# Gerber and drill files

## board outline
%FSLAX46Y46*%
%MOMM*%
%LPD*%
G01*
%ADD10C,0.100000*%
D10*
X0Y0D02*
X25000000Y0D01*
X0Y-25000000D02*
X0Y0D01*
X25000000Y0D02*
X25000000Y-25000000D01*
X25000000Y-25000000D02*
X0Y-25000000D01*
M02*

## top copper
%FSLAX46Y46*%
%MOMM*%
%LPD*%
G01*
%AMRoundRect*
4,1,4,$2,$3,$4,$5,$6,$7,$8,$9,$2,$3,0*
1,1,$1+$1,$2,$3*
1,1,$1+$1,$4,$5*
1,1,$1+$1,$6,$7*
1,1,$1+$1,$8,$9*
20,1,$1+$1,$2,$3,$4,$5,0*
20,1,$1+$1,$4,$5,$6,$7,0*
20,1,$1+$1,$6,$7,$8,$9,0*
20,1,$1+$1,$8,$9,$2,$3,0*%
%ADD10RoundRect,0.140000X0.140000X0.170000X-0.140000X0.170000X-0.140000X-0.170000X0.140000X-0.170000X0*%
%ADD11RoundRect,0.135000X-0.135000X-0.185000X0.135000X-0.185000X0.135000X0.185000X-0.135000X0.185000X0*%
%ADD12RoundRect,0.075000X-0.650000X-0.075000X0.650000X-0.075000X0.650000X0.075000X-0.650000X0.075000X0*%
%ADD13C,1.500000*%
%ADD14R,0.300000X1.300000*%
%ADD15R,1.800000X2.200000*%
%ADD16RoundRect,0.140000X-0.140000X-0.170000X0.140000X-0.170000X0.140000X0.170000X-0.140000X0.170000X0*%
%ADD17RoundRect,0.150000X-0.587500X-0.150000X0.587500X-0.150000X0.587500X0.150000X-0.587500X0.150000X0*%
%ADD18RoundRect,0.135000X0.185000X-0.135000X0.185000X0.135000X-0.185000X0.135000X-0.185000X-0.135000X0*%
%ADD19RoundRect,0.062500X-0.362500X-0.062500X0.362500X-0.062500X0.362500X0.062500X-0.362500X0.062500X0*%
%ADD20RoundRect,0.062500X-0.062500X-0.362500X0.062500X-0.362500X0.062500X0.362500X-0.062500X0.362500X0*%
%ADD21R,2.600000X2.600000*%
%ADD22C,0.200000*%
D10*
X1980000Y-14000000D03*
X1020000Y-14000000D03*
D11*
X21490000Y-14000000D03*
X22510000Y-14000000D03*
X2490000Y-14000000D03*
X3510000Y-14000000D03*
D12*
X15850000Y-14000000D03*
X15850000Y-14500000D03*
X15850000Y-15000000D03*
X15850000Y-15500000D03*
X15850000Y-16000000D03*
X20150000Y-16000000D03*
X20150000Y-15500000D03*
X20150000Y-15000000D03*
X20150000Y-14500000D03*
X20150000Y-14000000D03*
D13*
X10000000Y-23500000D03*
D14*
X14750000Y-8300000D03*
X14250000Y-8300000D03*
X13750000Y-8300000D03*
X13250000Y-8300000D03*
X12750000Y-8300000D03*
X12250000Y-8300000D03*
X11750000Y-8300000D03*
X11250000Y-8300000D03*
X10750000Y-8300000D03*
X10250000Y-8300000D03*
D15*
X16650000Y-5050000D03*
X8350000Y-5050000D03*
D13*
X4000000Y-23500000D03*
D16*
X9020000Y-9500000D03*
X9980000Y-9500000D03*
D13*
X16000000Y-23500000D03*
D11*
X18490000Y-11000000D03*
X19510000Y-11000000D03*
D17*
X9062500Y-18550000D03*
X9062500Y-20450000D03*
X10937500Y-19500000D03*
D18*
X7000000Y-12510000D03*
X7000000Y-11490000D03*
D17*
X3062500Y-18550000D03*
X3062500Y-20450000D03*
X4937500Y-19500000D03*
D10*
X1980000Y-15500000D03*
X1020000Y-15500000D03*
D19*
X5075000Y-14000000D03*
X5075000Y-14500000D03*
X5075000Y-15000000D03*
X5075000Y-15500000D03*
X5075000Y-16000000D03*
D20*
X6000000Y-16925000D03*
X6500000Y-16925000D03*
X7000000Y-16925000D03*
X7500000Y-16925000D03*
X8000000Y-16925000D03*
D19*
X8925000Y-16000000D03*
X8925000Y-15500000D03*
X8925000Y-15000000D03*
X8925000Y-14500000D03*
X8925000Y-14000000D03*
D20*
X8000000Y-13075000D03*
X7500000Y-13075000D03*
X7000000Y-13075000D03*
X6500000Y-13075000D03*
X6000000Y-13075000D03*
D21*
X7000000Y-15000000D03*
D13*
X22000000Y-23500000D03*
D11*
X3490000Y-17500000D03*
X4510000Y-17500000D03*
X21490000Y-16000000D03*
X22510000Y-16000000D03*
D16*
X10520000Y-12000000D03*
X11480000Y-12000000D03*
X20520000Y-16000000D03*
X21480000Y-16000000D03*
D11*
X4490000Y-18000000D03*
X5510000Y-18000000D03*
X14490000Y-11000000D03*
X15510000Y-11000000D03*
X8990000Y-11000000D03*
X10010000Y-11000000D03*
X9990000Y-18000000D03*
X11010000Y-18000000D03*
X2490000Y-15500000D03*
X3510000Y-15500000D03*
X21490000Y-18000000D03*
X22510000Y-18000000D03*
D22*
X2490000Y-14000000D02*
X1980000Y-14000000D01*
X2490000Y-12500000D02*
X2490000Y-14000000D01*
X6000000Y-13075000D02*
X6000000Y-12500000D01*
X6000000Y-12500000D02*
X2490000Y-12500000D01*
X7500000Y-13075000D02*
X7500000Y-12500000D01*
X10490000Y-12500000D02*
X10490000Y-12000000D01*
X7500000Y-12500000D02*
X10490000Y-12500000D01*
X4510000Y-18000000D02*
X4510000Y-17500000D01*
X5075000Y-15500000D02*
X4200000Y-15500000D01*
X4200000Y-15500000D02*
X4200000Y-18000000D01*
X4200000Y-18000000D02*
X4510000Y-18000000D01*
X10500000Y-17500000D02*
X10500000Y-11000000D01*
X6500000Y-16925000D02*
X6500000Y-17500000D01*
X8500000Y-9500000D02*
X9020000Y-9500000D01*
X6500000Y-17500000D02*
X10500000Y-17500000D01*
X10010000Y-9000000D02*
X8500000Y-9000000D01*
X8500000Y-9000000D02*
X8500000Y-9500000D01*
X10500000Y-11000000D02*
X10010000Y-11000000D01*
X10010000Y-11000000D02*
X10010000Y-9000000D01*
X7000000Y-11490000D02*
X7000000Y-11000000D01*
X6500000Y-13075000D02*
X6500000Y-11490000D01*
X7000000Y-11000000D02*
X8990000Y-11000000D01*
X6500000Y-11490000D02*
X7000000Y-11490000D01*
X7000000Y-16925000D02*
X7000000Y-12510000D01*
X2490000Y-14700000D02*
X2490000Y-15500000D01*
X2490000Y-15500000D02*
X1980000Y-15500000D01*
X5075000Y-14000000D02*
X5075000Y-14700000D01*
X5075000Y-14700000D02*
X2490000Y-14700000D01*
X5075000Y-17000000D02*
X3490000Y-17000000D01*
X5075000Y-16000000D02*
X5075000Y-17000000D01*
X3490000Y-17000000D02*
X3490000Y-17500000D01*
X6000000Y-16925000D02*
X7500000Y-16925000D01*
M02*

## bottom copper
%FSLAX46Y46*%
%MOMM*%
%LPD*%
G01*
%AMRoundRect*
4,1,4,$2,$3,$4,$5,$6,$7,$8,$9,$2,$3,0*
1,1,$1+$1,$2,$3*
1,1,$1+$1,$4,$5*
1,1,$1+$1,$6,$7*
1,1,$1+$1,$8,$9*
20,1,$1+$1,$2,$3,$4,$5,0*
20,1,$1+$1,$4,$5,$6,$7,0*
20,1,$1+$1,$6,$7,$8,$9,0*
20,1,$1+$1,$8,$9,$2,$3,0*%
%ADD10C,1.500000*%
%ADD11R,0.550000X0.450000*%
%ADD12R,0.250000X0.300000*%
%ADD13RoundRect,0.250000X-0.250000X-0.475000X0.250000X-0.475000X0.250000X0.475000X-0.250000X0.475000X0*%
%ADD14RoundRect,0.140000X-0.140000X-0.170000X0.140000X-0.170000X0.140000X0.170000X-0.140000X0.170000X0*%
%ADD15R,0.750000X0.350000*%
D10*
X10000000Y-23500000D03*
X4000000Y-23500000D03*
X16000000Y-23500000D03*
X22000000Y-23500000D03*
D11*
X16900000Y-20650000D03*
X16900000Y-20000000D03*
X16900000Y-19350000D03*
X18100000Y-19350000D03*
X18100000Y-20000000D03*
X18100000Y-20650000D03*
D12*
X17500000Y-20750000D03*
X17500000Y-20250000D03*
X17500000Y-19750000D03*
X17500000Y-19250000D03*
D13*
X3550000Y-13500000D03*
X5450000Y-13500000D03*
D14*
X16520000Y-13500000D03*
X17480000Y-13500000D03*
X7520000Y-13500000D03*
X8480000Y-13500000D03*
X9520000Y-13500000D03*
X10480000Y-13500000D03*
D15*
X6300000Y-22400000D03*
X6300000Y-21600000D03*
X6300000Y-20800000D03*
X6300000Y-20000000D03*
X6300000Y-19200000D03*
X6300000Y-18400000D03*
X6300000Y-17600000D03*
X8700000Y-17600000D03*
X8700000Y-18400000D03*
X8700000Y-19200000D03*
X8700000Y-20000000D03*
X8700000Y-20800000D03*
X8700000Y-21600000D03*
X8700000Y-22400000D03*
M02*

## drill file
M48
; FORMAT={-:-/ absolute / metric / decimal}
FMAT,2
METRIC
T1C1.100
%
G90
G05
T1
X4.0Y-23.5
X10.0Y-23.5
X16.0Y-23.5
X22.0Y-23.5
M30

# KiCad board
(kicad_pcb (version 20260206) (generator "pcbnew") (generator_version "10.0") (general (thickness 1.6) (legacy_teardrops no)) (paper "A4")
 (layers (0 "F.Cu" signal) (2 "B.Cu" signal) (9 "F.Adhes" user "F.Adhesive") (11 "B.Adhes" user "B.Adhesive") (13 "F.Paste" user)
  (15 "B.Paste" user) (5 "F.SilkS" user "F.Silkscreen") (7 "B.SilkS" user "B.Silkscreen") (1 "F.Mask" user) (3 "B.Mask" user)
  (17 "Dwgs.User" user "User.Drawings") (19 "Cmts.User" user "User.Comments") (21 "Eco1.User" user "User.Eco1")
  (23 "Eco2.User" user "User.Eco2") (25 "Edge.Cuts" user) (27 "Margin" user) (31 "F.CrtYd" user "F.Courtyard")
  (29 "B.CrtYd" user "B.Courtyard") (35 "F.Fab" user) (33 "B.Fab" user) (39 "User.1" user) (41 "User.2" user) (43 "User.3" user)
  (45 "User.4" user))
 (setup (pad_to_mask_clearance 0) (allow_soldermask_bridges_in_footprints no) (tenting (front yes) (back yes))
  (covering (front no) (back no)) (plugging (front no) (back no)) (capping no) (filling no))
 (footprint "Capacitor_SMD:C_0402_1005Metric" (layer "F.Cu") (at 1.5 14 180)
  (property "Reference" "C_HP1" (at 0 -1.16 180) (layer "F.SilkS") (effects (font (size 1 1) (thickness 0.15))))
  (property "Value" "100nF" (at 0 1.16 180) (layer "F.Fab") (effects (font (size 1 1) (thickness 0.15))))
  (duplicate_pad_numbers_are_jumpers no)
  (pad "1" smd roundrect (at -0.48 0 180) (size 0.56 0.62) (layers "F.Cu" "F.Mask" "F.Paste") (roundrect_rratio 0.25) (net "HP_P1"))
  (pad "2" smd roundrect (at 0.48 0 180) (size 0.56 0.62) (layers "F.Cu" "F.Mask" "F.Paste") (roundrect_rratio 0.25) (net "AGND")))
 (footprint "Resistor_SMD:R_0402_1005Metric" (layer "F.Cu") (at 22 14)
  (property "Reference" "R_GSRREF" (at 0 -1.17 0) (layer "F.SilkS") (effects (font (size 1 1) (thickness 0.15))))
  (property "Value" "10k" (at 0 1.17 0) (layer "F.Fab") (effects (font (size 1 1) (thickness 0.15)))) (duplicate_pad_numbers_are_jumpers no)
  (pad "1" smd roundrect (at -0.51 0) (size 0.54 0.64) (layers "F.Cu" "F.Mask" "F.Paste") (roundrect_rratio 0.25) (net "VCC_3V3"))
  (pad "2" smd roundrect (at 0.51 0) (size 0.54 0.64) (layers "F.Cu" "F.Mask" "F.Paste") (roundrect_rratio 0.25) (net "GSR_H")))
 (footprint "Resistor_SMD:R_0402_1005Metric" (layer "F.Cu") (at 3 14)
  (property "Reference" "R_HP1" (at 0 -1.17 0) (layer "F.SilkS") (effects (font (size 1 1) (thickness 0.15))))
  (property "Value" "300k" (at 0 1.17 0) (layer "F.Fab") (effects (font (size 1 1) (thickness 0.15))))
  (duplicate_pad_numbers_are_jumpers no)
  (pad "1" smd roundrect (at -0.51 0) (size 0.54 0.64) (layers "F.Cu" "F.Mask" "F.Paste") (roundrect_rratio 0.25) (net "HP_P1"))
  (pad "2" smd roundrect (at 0.51 0) (size 0.54 0.64) (layers "F.Cu" "F.Mask" "F.Paste") (roundrect_rratio 0.25) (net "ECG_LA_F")))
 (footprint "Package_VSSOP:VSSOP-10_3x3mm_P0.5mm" (layer "F.Cu") (at 18 15)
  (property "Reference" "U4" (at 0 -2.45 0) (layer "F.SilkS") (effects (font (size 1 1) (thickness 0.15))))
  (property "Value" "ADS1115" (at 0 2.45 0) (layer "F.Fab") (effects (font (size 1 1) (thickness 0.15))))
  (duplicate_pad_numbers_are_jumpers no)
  (pad "1" smd roundrect (at -2.15 -1) (size 1.45 0.3) (layers "F.Cu" "F.Mask" "F.Paste") (roundrect_rratio 0.25) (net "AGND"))
  (pad "2" smd roundrect (at -2.15 -0.5) (size 1.45 0.3) (layers "F.Cu" "F.Mask" "F.Paste") (roundrect_rratio 0.25))
  (pad "3" smd roundrect (at -2.15 0) (size 1.45 0.3) (layers "F.Cu" "F.Mask" "F.Paste") (roundrect_rratio 0.25) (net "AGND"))
  (pad "4" smd roundrect (at -2.15 0.5) (size 1.45 0.3) (layers "F.Cu" "F.Mask" "F.Paste") (roundrect_rratio 0.25) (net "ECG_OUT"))
  (pad "5" smd roundrect (at -2.15 1) (size 1.45 0.3) (layers "F.Cu" "F.Mask" "F.Paste") (roundrect_rratio 0.25) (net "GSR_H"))
  (pad "6" smd roundrect (at 2.15 1) (size 1.45 0.3) (layers "F.Cu" "F.Mask" "F.Paste") (roundrect_rratio 0.25) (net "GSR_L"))
  (pad "7" smd roundrect (at 2.15 0.5) (size 1.45 0.3) (layers "F.Cu" "F.Mask" "F.Paste") (roundrect_rratio 0.25))
  (pad "8" smd roundrect (at 2.15 0) (size 1.45 0.3) (layers "F.Cu" "F.Mask" "F.Paste") (roundrect_rratio 0.25) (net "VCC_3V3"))
  (pad "9" smd roundrect (at 2.15 -0.5) (size 1.45 0.3) (layers "F.Cu" "F.Mask" "F.Paste") (roundrect_rratio 0.25) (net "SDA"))
  (pad "10" smd roundrect (at 2.15 -1) (size 1.45 0.3) (layers "F.Cu" "F.Mask" "F.Paste") (roundrect_rratio 0.25) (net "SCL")))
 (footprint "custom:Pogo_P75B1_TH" (layer "F.Cu") (at 10 23.5)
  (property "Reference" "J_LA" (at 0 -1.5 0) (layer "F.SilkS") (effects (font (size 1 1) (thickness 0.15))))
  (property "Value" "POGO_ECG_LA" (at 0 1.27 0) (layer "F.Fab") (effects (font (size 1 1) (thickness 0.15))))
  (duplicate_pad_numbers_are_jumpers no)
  (pad "1" thru_hole circle (at 0 0) (size 1.5 1.5) (drill 1.1) (layers "*.Cu" "*.Mask") (remove_unused_layers no) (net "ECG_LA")))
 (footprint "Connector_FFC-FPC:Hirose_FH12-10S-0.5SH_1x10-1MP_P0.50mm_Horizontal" (layer "F.Cu") (at 12.5 6.45 180)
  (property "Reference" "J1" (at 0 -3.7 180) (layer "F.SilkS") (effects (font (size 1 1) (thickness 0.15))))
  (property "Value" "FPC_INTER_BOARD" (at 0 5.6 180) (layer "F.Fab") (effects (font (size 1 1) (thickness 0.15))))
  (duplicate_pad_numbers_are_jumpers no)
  (pad "1" smd rect (at -2.25 -1.85 180) (size 0.3 1.3) (layers "F.Cu" "F.Mask" "F.Paste") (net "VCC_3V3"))
  (pad "2" smd rect (at -1.75 -1.85 180) (size 0.3 1.3) (layers "F.Cu" "F.Mask" "F.Paste") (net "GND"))
  (pad "3" smd rect (at -1.25 -1.85 180) (size 0.3 1.3) (layers "F.Cu" "F.Mask" "F.Paste") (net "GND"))
  (pad "4" smd rect (at -0.75 -1.85 180) (size 0.3 1.3) (layers "F.Cu" "F.Mask" "F.Paste") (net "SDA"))
  (pad "5" smd rect (at -0.25 -1.85 180) (size 0.3 1.3) (layers "F.Cu" "F.Mask" "F.Paste") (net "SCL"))
  (pad "6" smd rect (at 0.25 -1.85 180) (size 0.3 1.3) (layers "F.Cu" "F.Mask" "F.Paste") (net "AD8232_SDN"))
  (pad "7" smd rect (at 0.75 -1.85 180) (size 0.3 1.3) (layers "F.Cu" "F.Mask" "F.Paste") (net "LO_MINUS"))
  (pad "8" smd rect (at 1.25 -1.85 180) (size 0.3 1.3) (layers "F.Cu" "F.Mask" "F.Paste") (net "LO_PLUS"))
  (pad "9" smd rect (at 1.75 -1.85 180) (size 0.3 1.3) (layers "F.Cu" "F.Mask" "F.Paste") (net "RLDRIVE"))
  (pad "10" smd rect (at 2.25 -1.85 180) (size 0.3 1.3) (layers "F.Cu" "F.Mask" "F.Paste"))
  (pad "MP" smd rect (at -4.15 1.4 180) (size 1.8 2.2) (layers "F.Cu" "F.Mask" "F.Paste"))
  (pad "MP" smd rect (at 4.15 1.4 180) (size 1.8 2.2) (layers "F.Cu" "F.Mask" "F.Paste")))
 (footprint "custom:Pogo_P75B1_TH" (layer "F.Cu") (at 4 23.5)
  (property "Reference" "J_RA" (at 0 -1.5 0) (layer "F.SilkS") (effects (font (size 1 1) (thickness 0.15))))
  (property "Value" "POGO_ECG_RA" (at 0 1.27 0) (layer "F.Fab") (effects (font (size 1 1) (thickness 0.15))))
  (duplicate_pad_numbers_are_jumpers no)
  (pad "1" thru_hole circle (at 0 0) (size 1.5 1.5) (drill 1.1) (layers "*.Cu" "*.Mask") (remove_unused_layers no) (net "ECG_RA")))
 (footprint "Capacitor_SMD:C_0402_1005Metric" (layer "F.Cu") (at 9.5 9.5)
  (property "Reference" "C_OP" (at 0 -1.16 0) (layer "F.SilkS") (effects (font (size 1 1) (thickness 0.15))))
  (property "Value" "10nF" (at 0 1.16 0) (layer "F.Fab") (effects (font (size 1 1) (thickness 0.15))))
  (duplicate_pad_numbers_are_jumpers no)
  (pad "1" smd roundrect (at -0.48 0) (size 0.56 0.62) (layers "F.Cu" "F.Mask" "F.Paste") (roundrect_rratio 0.25) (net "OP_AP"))
  (pad "2" smd roundrect (at 0.48 0) (size 0.56 0.62) (layers "F.Cu" "F.Mask" "F.Paste") (roundrect_rratio 0.25) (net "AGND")))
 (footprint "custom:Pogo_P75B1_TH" (layer "F.Cu") (at 16 23.5)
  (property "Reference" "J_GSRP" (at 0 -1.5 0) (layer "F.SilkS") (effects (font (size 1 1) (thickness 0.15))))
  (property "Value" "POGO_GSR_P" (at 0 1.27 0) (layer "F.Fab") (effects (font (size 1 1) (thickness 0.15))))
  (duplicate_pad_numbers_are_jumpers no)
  (pad "1" thru_hole circle (at 0 0) (size 1.5 1.5) (drill 1.1) (layers "*.Cu" "*.Mask") (remove_unused_layers no) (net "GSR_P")))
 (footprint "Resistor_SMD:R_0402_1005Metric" (layer "F.Cu") (at 19 11)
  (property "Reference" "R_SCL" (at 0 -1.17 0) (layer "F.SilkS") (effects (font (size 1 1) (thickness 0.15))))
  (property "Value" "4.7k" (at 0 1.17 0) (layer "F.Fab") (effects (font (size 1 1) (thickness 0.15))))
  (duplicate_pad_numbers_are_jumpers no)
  (pad "1" smd roundrect (at -0.51 0) (size 0.54 0.64) (layers "F.Cu" "F.Mask" "F.Paste") (roundrect_rratio 0.25) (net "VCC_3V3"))
  (pad "2" smd roundrect (at 0.51 0) (size 0.54 0.64) (layers "F.Cu" "F.Mask" "F.Paste") (roundrect_rratio 0.25) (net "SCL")))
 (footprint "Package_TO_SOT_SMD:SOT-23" (layer "F.Cu") (at 10 19.5)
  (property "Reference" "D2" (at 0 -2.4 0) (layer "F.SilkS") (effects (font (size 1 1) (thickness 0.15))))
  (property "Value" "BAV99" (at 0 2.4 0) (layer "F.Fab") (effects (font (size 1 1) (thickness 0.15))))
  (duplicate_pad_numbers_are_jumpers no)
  (pad "1" smd roundrect (at -0.9375 -0.95) (size 1.475 0.6) (layers "F.Cu" "F.Mask" "F.Paste") (roundrect_rratio 0.25) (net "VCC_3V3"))
  (pad "2" smd roundrect (at -0.9375 0.95) (size 1.475 0.6) (layers "F.Cu" "F.Mask" "F.Paste") (roundrect_rratio 0.25) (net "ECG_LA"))
  (pad "3" smd roundrect (at 0.9375 0) (size 1.475 0.6) (layers "F.Cu" "F.Mask" "F.Paste") (roundrect_rratio 0.25) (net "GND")))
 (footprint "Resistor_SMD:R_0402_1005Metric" (layer "F.Cu") (at 7 12 90)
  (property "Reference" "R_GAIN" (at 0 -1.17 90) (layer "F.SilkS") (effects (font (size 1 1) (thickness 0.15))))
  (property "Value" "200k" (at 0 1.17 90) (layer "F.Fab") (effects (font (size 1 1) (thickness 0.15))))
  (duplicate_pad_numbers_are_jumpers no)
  (pad "1" smd roundrect (at -0.51 0 90) (size 0.54 0.64) (layers "F.Cu" "F.Mask" "F.Paste") (roundrect_rratio 0.25) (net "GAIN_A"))
  (pad "2" smd roundrect (at 0.51 0 90) (size 0.54 0.64) (layers "F.Cu" "F.Mask" "F.Paste") (roundrect_rratio 0.25) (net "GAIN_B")))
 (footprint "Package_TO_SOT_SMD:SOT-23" (layer "F.Cu") (at 4 19.5)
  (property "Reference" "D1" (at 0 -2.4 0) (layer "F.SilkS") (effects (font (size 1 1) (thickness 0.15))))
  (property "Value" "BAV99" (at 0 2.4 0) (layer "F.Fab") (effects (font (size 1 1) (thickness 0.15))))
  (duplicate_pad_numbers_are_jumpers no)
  (pad "1" smd roundrect (at -0.9375 -0.95) (size 1.475 0.6) (layers "F.Cu" "F.Mask" "F.Paste") (roundrect_rratio 0.25) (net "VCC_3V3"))
  (pad "2" smd roundrect (at -0.9375 0.95) (size 1.475 0.6) (layers "F.Cu" "F.Mask" "F.Paste") (roundrect_rratio 0.25) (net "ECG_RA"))
  (pad "3" smd roundrect (at 0.9375 0) (size 1.475 0.6) (layers "F.Cu" "F.Mask" "F.Paste") (roundrect_rratio 0.25) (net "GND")))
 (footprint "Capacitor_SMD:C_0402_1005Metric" (layer "F.Cu") (at 1.5 15.5 180)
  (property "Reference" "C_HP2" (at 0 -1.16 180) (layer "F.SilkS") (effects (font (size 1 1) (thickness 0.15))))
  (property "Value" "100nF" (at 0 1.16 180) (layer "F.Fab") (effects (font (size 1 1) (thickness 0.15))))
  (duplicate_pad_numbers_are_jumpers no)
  (pad "1" smd roundrect (at -0.48 0 180) (size 0.56 0.62) (layers "F.Cu" "F.Mask" "F.Paste") (roundrect_rratio 0.25) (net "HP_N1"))
  (pad "2" smd roundrect (at 0.48 0 180) (size 0.56 0.62) (layers "F.Cu" "F.Mask" "F.Paste") (roundrect_rratio 0.25) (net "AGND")))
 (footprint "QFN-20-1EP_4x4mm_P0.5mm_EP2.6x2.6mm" (layer "F.Cu") (at 7 15)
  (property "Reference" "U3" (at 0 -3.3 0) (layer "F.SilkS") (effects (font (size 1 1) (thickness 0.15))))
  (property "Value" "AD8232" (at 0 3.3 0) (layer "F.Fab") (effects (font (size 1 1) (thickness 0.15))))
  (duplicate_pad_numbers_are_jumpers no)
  (pad "" smd roundrect (at -0.65 -0.65) (size 1.05 1.05) (layers "F.Paste") (roundrect_rratio 0.238095))
  (pad "" smd roundrect (at -0.65 0.65) (size 1.05 1.05) (layers "F.Paste") (roundrect_rratio 0.238095))
  (pad "" smd roundrect (at 0.65 -0.65) (size 1.05 1.05) (layers "F.Paste") (roundrect_rratio 0.238095))
  (pad "" smd roundrect (at 0.65 0.65) (size 1.05 1.05) (layers "F.Paste") (roundrect_rratio 0.238095))
  (pad "1" smd roundrect (at -1.925 -1) (size 0.85 0.25) (layers "F.Cu" "F.Mask" "F.Paste") (roundrect_rratio 0.25) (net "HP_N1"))
  (pad "2" smd roundrect (at -1.925 -0.5) (size 0.85 0.25) (layers "F.Cu" "F.Mask" "F.Paste") (roundrect_rratio 0.25) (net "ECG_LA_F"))
  (pad "3" smd roundrect (at -1.925 0) (size 0.85 0.25) (layers "F.Cu" "F.Mask" "F.Paste") (roundrect_rratio 0.25) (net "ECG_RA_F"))
  (pad "4" smd roundrect (at -1.925 0.5) (size 0.85 0.25) (layers "F.Cu" "F.Mask" "F.Paste") (roundrect_rratio 0.25) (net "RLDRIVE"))
  (pad "5" smd roundrect (at -1.925 1) (size 0.85 0.25) (layers "F.Cu" "F.Mask" "F.Paste") (roundrect_rratio 0.25) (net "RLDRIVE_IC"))
  (pad "6" smd roundrect (at -1 1.925) (size 0.25 0.85) (layers "F.Cu" "F.Mask" "F.Paste") (roundrect_rratio 0.25) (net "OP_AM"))
  (pad "7" smd roundrect (at -0.5 1.925) (size 0.25 0.85) (layers "F.Cu" "F.Mask" "F.Paste") (roundrect_rratio 0.25) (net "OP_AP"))
  (pad "8" smd roundrect (at 0 1.925) (size 0.25 0.85) (layers "F.Cu" "F.Mask" "F.Paste") (roundrect_rratio 0.25) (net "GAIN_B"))
  (pad "9" smd roundrect (at 0.5 1.925) (size 0.25 0.85) (layers "F.Cu" "F.Mask" "F.Paste") (roundrect_rratio 0.25) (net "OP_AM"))
  (pad "10" smd roundrect (at 1 1.925) (size 0.25 0.85) (layers "F.Cu" "F.Mask" "F.Paste") (roundrect_rratio 0.25) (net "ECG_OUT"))
  (pad "11" smd roundrect (at 1.925 1) (size 0.85 0.25) (layers "F.Cu" "F.Mask" "F.Paste") (roundrect_rratio 0.25) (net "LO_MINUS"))
  (pad "12" smd roundrect (at 1.925 0.5) (size 0.85 0.25) (layers "F.Cu" "F.Mask" "F.Paste") (roundrect_rratio 0.25) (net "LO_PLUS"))
  (pad "13" smd roundrect (at 1.925 0) (size 0.85 0.25) (layers "F.Cu" "F.Mask" "F.Paste") (roundrect_rratio 0.25) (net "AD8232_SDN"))
  (pad "14" smd roundrect (at 1.925 -0.5) (size 0.85 0.25) (layers "F.Cu" "F.Mask" "F.Paste") (roundrect_rratio 0.25) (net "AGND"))
  (pad "15" smd roundrect (at 1.925 -1) (size 0.85 0.25) (layers "F.Cu" "F.Mask" "F.Paste") (roundrect_rratio 0.25) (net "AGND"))
  (pad "16" smd roundrect (at 1 -1.925) (size 0.25 0.85) (layers "F.Cu" "F.Mask" "F.Paste") (roundrect_rratio 0.25) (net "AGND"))
  (pad "17" smd roundrect (at 0.5 -1.925) (size 0.25 0.85) (layers "F.Cu" "F.Mask" "F.Paste") (roundrect_rratio 0.25) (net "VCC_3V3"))
  (pad "18" smd roundrect (at 0 -1.925) (size 0.25 0.85) (layers "F.Cu" "F.Mask" "F.Paste") (roundrect_rratio 0.25) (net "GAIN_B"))
  (pad "19" smd roundrect (at -0.5 -1.925) (size 0.25 0.85) (layers "F.Cu" "F.Mask" "F.Paste") (roundrect_rratio 0.25) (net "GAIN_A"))
  (pad "20" smd roundrect (at -1 -1.925) (size 0.25 0.85) (layers "F.Cu" "F.Mask" "F.Paste") (roundrect_rratio 0.25) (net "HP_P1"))
  (pad "21" smd rect (at 0 0) (size 2.6 2.6) (layers "F.Cu" "F.Mask") (zone_connect 2)))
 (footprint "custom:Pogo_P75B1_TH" (layer "F.Cu") (at 22 23.5)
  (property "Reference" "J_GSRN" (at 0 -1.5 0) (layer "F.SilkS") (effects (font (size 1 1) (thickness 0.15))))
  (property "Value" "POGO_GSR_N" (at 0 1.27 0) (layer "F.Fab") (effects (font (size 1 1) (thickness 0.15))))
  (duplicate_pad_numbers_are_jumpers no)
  (pad "1" thru_hole circle (at 0 0) (size 1.5 1.5) (drill 1.1) (layers "*.Cu" "*.Mask") (remove_unused_layers no) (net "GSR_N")))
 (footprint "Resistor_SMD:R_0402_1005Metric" (layer "F.Cu") (at 4 17.5)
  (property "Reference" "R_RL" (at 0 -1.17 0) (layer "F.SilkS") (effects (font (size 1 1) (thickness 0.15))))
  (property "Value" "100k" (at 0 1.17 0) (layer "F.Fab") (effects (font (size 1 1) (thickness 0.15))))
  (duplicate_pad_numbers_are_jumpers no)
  (pad "1" smd roundrect (at -0.51 0) (size 0.54 0.64) (layers "F.Cu" "F.Mask" "F.Paste") (roundrect_rratio 0.25) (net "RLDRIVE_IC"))
  (pad "2" smd roundrect (at 0.51 0) (size 0.54 0.64) (layers "F.Cu" "F.Mask" "F.Paste") (roundrect_rratio 0.25) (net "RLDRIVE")))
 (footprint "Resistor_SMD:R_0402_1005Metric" (layer "F.Cu") (at 22 16)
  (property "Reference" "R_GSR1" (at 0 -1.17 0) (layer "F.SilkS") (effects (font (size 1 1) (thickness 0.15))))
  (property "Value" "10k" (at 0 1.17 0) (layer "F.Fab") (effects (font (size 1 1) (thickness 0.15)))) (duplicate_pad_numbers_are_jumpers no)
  (pad "1" smd roundrect (at -0.51 0) (size 0.54 0.64) (layers "F.Cu" "F.Mask" "F.Paste") (roundrect_rratio 0.25) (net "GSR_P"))
  (pad "2" smd roundrect (at 0.51 0) (size 0.54 0.64) (layers "F.Cu" "F.Mask" "F.Paste") (roundrect_rratio 0.25) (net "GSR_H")))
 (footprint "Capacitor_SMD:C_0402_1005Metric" (layer "F.Cu") (at 11 12)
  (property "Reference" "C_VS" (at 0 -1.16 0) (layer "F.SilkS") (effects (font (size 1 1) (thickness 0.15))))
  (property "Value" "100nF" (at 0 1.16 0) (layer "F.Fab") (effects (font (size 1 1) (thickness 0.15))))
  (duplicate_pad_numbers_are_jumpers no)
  (pad "1" smd roundrect (at -0.48 0) (size 0.56 0.62) (layers "F.Cu" "F.Mask" "F.Paste") (roundrect_rratio 0.25) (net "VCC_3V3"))
  (pad "2" smd roundrect (at 0.48 0) (size 0.56 0.62) (layers "F.Cu" "F.Mask" "F.Paste") (roundrect_rratio 0.25) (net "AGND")))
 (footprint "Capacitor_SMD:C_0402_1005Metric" (layer "F.Cu") (at 21 16)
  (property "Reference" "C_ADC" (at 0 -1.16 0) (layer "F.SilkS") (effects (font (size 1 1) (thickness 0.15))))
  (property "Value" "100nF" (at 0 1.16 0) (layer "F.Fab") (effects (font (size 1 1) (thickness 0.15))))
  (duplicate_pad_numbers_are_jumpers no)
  (pad "1" smd roundrect (at -0.48 0) (size 0.56 0.62) (layers "F.Cu" "F.Mask" "F.Paste") (roundrect_rratio 0.25) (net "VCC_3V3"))
  (pad "2" smd roundrect (at 0.48 0) (size 0.56 0.62) (layers "F.Cu" "F.Mask" "F.Paste") (roundrect_rratio 0.25) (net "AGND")))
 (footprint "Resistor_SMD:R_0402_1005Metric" (layer "F.Cu") (at 5 18)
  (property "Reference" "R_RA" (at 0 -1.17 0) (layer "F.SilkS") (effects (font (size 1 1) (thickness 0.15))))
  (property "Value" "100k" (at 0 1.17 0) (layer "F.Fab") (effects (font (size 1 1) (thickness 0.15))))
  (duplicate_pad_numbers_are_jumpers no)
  (pad "1" smd roundrect (at -0.51 0) (size 0.54 0.64) (layers "F.Cu" "F.Mask" "F.Paste") (roundrect_rratio 0.25) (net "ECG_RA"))
  (pad "2" smd roundrect (at 0.51 0) (size 0.54 0.64) (layers "F.Cu" "F.Mask" "F.Paste") (roundrect_rratio 0.25) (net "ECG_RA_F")))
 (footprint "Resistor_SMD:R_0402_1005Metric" (layer "F.Cu") (at 15 11)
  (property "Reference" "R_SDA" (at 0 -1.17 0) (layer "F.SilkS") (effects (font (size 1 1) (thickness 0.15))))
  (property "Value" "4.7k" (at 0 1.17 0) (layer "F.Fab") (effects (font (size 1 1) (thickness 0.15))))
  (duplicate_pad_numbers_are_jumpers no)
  (pad "1" smd roundrect (at -0.51 0) (size 0.54 0.64) (layers "F.Cu" "F.Mask" "F.Paste") (roundrect_rratio 0.25) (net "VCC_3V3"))
  (pad "2" smd roundrect (at 0.51 0) (size 0.54 0.64) (layers "F.Cu" "F.Mask" "F.Paste") (roundrect_rratio 0.25) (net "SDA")))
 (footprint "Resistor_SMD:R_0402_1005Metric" (layer "F.Cu") (at 9.5 11)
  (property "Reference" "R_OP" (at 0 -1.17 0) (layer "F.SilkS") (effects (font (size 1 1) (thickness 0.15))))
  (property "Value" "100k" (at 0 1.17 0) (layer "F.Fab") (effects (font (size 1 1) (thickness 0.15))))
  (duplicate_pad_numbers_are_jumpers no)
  (pad "1" smd roundrect (at -0.51 0) (size 0.54 0.64) (layers "F.Cu" "F.Mask" "F.Paste") (roundrect_rratio 0.25) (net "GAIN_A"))
  (pad "2" smd roundrect (at 0.51 0) (size 0.54 0.64) (layers "F.Cu" "F.Mask" "F.Paste") (roundrect_rratio 0.25) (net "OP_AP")))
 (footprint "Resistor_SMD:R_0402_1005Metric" (layer "F.Cu") (at 10.5 18)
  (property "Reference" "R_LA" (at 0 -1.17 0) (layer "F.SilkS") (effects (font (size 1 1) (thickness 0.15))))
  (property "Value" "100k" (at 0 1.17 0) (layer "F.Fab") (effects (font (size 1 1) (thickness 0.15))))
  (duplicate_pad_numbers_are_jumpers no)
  (pad "1" smd roundrect (at -0.51 0) (size 0.54 0.64) (layers "F.Cu" "F.Mask" "F.Paste") (roundrect_rratio 0.25) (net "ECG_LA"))
  (pad "2" smd roundrect (at 0.51 0) (size 0.54 0.64) (layers "F.Cu" "F.Mask" "F.Paste") (roundrect_rratio 0.25) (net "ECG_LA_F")))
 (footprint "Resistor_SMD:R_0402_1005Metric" (layer "F.Cu") (at 3 15.5)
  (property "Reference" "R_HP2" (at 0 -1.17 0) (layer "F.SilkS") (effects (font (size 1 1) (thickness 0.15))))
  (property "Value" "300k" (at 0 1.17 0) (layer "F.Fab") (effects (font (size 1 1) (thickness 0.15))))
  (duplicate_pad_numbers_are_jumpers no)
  (pad "1" smd roundrect (at -0.51 0) (size 0.54 0.64) (layers "F.Cu" "F.Mask" "F.Paste") (roundrect_rratio 0.25) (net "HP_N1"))
  (pad "2" smd roundrect (at 0.51 0) (size 0.54 0.64) (layers "F.Cu" "F.Mask" "F.Paste") (roundrect_rratio 0.25) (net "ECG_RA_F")))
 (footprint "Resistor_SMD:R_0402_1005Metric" (layer "F.Cu") (at 22 18)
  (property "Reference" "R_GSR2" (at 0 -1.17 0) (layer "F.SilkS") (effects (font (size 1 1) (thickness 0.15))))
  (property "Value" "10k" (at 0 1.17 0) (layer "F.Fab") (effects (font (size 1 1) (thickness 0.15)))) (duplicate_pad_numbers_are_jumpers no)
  (pad "1" smd roundrect (at -0.51 0) (size 0.54 0.64) (layers "F.Cu" "F.Mask" "F.Paste") (roundrect_rratio 0.25) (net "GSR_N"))
  (pad "2" smd roundrect (at 0.51 0) (size 0.54 0.64) (layers "F.Cu" "F.Mask" "F.Paste") (roundrect_rratio 0.25) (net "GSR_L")))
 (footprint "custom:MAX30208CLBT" (layer "B.Cu") (at 17.5 20)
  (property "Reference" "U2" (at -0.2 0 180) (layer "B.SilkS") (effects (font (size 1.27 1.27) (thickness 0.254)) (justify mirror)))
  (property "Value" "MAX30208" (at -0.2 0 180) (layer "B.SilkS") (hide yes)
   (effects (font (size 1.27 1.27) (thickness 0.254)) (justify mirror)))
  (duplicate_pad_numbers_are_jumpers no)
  (pad "1" smd rect (at -0.6 0.65 270) (size 0.45 0.55) (layers "B.Cu" "B.Mask" "B.Paste") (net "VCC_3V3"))
  (pad "2" smd rect (at -0.6 0 270) (size 0.45 0.55) (layers "B.Cu" "B.Mask" "B.Paste") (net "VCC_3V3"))
  (pad "3" smd rect (at -0.6 -0.65 270) (size 0.45 0.55) (layers "B.Cu" "B.Mask" "B.Paste") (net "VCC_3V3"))
  (pad "4" smd rect (at 0.6 -0.65 270) (size 0.45 0.55) (layers "B.Cu" "B.Mask" "B.Paste") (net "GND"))
  (pad "5" smd rect (at 0.6 0 270) (size 0.45 0.55) (layers "B.Cu" "B.Mask" "B.Paste") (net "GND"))
  (pad "6" smd rect (at 0.6 0.65 270) (size 0.45 0.55) (layers "B.Cu" "B.Mask" "B.Paste") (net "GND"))
  (pad "7" smd rect (at 0 0.75) (size 0.25 0.3) (layers "B.Cu" "B.Mask" "B.Paste") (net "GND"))
  (pad "8" smd rect (at 0 0.25) (size 0.25 0.3) (layers "B.Cu" "B.Mask" "B.Paste") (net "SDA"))
  (pad "9" smd rect (at 0 -0.25) (size 0.25 0.3) (layers "B.Cu" "B.Mask" "B.Paste") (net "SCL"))
  (pad "10" smd rect (at 0 -0.75) (size 0.25 0.3) (layers "B.Cu" "B.Mask" "B.Paste") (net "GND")))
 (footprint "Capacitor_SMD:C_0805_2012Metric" (layer "B.Cu") (at 4.5 13.5)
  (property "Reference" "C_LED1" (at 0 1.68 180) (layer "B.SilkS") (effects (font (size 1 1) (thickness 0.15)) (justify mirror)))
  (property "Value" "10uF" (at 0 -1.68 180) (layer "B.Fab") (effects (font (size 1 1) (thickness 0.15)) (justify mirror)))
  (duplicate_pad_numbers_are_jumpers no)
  (pad "1" smd roundrect (at -0.95 0) (size 1 1.45) (layers "B.Cu" "B.Mask" "B.Paste") (roundrect_rratio 0.25) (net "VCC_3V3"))
  (pad "2" smd roundrect (at 0.95 0) (size 1 1.45) (layers "B.Cu" "B.Mask" "B.Paste") (roundrect_rratio 0.25) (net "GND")))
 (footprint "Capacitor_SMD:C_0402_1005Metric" (layer "B.Cu") (at 17 13.5)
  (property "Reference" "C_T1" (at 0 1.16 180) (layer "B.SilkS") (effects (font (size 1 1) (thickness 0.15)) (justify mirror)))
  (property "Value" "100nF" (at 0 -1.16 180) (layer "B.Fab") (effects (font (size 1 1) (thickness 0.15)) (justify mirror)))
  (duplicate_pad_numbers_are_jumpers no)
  (pad "1" smd roundrect (at -0.48 0) (size 0.56 0.62) (layers "B.Cu" "B.Mask" "B.Paste") (roundrect_rratio 0.25) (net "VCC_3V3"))
  (pad "2" smd roundrect (at 0.48 0) (size 0.56 0.62) (layers "B.Cu" "B.Mask" "B.Paste") (roundrect_rratio 0.25) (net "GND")))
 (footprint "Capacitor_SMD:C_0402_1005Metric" (layer "B.Cu") (at 8 13.5)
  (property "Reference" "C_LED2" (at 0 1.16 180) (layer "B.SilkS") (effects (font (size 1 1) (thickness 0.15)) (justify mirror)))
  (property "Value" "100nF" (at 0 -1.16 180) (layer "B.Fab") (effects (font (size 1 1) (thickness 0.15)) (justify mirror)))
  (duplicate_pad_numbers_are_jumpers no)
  (pad "1" smd roundrect (at -0.48 0) (size 0.56 0.62) (layers "B.Cu" "B.Mask" "B.Paste") (roundrect_rratio 0.25) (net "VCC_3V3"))
  (pad "2" smd roundrect (at 0.48 0) (size 0.56 0.62) (layers "B.Cu" "B.Mask" "B.Paste") (roundrect_rratio 0.25) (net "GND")))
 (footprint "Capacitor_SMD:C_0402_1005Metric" (layer "B.Cu") (at 10 13.5)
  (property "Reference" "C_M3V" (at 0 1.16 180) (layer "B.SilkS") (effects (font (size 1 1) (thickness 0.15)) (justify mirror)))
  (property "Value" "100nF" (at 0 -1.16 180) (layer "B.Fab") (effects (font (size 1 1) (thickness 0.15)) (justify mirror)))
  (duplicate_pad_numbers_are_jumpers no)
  (pad "1" smd roundrect (at -0.48 0) (size 0.56 0.62) (layers "B.Cu" "B.Mask" "B.Paste") (roundrect_rratio 0.25) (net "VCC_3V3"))
  (pad "2" smd roundrect (at 0.48 0) (size 0.56 0.62) (layers "B.Cu" "B.Mask" "B.Paste") (roundrect_rratio 0.25) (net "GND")))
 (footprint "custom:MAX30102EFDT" (layer "B.Cu") (at 7.5 20)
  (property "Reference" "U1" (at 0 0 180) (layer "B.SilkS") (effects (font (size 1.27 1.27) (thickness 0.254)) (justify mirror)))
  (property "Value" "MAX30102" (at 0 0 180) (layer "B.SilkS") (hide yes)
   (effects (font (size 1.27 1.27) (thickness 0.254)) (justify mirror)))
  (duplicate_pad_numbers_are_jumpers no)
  (pad "1" smd rect (at -1.2 2.4 270) (size 0.35 0.75) (layers "B.Cu" "B.Mask" "B.Paste"))
  (pad "2" smd rect (at -1.2 1.6 270) (size 0.35 0.75) (layers "B.Cu" "B.Mask" "B.Paste") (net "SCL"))
  (pad "3" smd rect (at -1.2 0.8 270) (size 0.35 0.75) (layers "B.Cu" "B.Mask" "B.Paste") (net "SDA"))
  (pad "4" smd rect (at -1.2 0 270) (size 0.35 0.75) (layers "B.Cu" "B.Mask" "B.Paste") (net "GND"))
  (pad "5" smd rect (at -1.2 -0.8 270) (size 0.35 0.75) (layers "B.Cu" "B.Mask" "B.Paste"))
  (pad "6" smd rect (at -1.2 -1.6 270) (size 0.35 0.75) (layers "B.Cu" "B.Mask" "B.Paste"))
  (pad "7" smd rect (at -1.2 -2.4 270) (size 0.35 0.75) (layers "B.Cu" "B.Mask" "B.Paste"))
  (pad "8" smd rect (at 1.2 -2.4 270) (size 0.35 0.75) (layers "B.Cu" "B.Mask" "B.Paste"))
  (pad "9" smd rect (at 1.2 -1.6 270) (size 0.35 0.75) (layers "B.Cu" "B.Mask" "B.Paste") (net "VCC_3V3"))
  (pad "10" smd rect (at 1.2 -0.8 270) (size 0.35 0.75) (layers "B.Cu" "B.Mask" "B.Paste") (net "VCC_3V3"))
  (pad "11" smd rect (at 1.2 0 270) (size 0.35 0.75) (layers "B.Cu" "B.Mask" "B.Paste") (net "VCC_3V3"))
  (pad "12" smd rect (at 1.2 0.8 270) (size 0.35 0.75) (layers "B.Cu" "B.Mask" "B.Paste") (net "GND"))
  (pad "13" smd rect (at 1.2 1.6 270) (size 0.35 0.75) (layers "B.Cu" "B.Mask" "B.Paste"))
  (pad "14" smd rect (at 1.2 2.4 270) (size 0.35 0.75) (layers "B.Cu" "B.Mask" "B.Paste")))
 (gr_line (start 0 0) (end 25 0) (stroke (width 0.1) (type default)) (layer "Edge.Cuts"))
 (gr_line (start 0 25) (end 0 0) (stroke (width 0.1) (type default)) (layer "Edge.Cuts"))
 (gr_line (start 25 0) (end 25 25) (stroke (width 0.1) (type default)) (layer "Edge.Cuts"))
 (gr_line (start 25 25) (end 0 25) (stroke (width 0.1) (type default)) (layer "Edge.Cuts"))
 (segment (start 2.49 14) (end 1.98 14) (width 0.2) (layer "F.Cu") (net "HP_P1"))
 (segment (start 2.49 12.5) (end 2.49 14) (width 0.2) (layer "F.Cu") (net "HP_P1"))
 (segment (start 6 13.075) (end 6 12.5) (width 0.2) (layer "F.Cu") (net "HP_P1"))
 (segment (start 6 12.5) (end 2.49 12.5) (width 0.2) (layer "F.Cu") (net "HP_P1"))
 (segment (start 7.5 13.075) (end 7.5 12.5) (width 0.2) (layer "F.Cu") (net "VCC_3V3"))
 (segment (start 10.49 12.5) (end 10.49 12) (width 0.2) (layer "F.Cu") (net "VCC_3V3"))
 (segment (start 7.5 12.5) (end 10.49 12.5) (width 0.2) (layer "F.Cu") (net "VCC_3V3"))
 (segment (start 4.51 18) (end 4.51 17.5) (width 0.2) (layer "F.Cu") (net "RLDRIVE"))
 (segment (start 5.075 15.5) (end 4.2 15.5) (width 0.2) (layer "F.Cu") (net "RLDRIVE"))
 (segment (start 4.2 15.5) (end 4.2 18) (width 0.2) (layer "F.Cu") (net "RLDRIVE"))
 (segment (start 4.2 18) (end 4.51 18) (width 0.2) (layer "F.Cu") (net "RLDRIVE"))
 (segment (start 10.5 17.5) (end 10.5 11) (width 0.2) (layer "F.Cu") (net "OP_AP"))
 (segment (start 6.5 16.925) (end 6.5 17.5) (width 0.2) (layer "F.Cu") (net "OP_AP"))
 (segment (start 8.5 9.5) (end 9.02 9.5) (width 0.2) (layer "F.Cu") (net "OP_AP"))
 (segment (start 6.5 17.5) (end 10.5 17.5) (width 0.2) (layer "F.Cu") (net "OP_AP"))
 (segment (start 10.01 9) (end 8.5 9) (width 0.2) (layer "F.Cu") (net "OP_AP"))
 (segment (start 8.5 9) (end 8.5 9.5) (width 0.2) (layer "F.Cu") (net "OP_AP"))
 (segment (start 10.5 11) (end 10.01 11) (width 0.2) (layer "F.Cu") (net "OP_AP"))
 (segment (start 10.01 11) (end 10.01 9) (width 0.2) (layer "F.Cu") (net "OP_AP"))
 (segment (start 7 11.49) (end 7 11) (width 0.2) (layer "F.Cu") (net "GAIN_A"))
 (segment (start 6.5 13.075) (end 6.5 11.49) (width 0.2) (layer "F.Cu") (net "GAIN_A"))
 (segment (start 7 11) (end 8.99 11) (width 0.2) (layer "F.Cu") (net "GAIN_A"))
 (segment (start 6.5 11.49) (end 7 11.49) (width 0.2) (layer "F.Cu") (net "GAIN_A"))
 (segment (start 7 16.925) (end 7 12.51) (width 0.2) (layer "F.Cu") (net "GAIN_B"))
 (segment (start 2.49 14.7) (end 2.49 15.5) (width 0.2) (layer "F.Cu") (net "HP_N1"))
 (segment (start 2.49 15.5) (end 1.98 15.5) (width 0.2) (layer "F.Cu") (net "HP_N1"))
 (segment (start 5.075 14) (end 5.075 14.7) (width 0.2) (layer "F.Cu") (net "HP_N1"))
 (segment (start 5.075 14.7) (end 2.49 14.7) (width 0.2) (layer "F.Cu") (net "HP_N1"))
 (segment (start 5.075 17) (end 3.49 17) (width 0.2) (layer "F.Cu") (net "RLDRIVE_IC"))
 (segment (start 5.075 16) (end 5.075 17) (width 0.2) (layer "F.Cu") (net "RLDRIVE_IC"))
 (segment (start 3.49 17) (end 3.49 17.5) (width 0.2) (layer "F.Cu") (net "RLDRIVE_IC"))
 (segment (start 6 16.925) (end 7.5 16.925) (width 0.2) (layer "F.Cu") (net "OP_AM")))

